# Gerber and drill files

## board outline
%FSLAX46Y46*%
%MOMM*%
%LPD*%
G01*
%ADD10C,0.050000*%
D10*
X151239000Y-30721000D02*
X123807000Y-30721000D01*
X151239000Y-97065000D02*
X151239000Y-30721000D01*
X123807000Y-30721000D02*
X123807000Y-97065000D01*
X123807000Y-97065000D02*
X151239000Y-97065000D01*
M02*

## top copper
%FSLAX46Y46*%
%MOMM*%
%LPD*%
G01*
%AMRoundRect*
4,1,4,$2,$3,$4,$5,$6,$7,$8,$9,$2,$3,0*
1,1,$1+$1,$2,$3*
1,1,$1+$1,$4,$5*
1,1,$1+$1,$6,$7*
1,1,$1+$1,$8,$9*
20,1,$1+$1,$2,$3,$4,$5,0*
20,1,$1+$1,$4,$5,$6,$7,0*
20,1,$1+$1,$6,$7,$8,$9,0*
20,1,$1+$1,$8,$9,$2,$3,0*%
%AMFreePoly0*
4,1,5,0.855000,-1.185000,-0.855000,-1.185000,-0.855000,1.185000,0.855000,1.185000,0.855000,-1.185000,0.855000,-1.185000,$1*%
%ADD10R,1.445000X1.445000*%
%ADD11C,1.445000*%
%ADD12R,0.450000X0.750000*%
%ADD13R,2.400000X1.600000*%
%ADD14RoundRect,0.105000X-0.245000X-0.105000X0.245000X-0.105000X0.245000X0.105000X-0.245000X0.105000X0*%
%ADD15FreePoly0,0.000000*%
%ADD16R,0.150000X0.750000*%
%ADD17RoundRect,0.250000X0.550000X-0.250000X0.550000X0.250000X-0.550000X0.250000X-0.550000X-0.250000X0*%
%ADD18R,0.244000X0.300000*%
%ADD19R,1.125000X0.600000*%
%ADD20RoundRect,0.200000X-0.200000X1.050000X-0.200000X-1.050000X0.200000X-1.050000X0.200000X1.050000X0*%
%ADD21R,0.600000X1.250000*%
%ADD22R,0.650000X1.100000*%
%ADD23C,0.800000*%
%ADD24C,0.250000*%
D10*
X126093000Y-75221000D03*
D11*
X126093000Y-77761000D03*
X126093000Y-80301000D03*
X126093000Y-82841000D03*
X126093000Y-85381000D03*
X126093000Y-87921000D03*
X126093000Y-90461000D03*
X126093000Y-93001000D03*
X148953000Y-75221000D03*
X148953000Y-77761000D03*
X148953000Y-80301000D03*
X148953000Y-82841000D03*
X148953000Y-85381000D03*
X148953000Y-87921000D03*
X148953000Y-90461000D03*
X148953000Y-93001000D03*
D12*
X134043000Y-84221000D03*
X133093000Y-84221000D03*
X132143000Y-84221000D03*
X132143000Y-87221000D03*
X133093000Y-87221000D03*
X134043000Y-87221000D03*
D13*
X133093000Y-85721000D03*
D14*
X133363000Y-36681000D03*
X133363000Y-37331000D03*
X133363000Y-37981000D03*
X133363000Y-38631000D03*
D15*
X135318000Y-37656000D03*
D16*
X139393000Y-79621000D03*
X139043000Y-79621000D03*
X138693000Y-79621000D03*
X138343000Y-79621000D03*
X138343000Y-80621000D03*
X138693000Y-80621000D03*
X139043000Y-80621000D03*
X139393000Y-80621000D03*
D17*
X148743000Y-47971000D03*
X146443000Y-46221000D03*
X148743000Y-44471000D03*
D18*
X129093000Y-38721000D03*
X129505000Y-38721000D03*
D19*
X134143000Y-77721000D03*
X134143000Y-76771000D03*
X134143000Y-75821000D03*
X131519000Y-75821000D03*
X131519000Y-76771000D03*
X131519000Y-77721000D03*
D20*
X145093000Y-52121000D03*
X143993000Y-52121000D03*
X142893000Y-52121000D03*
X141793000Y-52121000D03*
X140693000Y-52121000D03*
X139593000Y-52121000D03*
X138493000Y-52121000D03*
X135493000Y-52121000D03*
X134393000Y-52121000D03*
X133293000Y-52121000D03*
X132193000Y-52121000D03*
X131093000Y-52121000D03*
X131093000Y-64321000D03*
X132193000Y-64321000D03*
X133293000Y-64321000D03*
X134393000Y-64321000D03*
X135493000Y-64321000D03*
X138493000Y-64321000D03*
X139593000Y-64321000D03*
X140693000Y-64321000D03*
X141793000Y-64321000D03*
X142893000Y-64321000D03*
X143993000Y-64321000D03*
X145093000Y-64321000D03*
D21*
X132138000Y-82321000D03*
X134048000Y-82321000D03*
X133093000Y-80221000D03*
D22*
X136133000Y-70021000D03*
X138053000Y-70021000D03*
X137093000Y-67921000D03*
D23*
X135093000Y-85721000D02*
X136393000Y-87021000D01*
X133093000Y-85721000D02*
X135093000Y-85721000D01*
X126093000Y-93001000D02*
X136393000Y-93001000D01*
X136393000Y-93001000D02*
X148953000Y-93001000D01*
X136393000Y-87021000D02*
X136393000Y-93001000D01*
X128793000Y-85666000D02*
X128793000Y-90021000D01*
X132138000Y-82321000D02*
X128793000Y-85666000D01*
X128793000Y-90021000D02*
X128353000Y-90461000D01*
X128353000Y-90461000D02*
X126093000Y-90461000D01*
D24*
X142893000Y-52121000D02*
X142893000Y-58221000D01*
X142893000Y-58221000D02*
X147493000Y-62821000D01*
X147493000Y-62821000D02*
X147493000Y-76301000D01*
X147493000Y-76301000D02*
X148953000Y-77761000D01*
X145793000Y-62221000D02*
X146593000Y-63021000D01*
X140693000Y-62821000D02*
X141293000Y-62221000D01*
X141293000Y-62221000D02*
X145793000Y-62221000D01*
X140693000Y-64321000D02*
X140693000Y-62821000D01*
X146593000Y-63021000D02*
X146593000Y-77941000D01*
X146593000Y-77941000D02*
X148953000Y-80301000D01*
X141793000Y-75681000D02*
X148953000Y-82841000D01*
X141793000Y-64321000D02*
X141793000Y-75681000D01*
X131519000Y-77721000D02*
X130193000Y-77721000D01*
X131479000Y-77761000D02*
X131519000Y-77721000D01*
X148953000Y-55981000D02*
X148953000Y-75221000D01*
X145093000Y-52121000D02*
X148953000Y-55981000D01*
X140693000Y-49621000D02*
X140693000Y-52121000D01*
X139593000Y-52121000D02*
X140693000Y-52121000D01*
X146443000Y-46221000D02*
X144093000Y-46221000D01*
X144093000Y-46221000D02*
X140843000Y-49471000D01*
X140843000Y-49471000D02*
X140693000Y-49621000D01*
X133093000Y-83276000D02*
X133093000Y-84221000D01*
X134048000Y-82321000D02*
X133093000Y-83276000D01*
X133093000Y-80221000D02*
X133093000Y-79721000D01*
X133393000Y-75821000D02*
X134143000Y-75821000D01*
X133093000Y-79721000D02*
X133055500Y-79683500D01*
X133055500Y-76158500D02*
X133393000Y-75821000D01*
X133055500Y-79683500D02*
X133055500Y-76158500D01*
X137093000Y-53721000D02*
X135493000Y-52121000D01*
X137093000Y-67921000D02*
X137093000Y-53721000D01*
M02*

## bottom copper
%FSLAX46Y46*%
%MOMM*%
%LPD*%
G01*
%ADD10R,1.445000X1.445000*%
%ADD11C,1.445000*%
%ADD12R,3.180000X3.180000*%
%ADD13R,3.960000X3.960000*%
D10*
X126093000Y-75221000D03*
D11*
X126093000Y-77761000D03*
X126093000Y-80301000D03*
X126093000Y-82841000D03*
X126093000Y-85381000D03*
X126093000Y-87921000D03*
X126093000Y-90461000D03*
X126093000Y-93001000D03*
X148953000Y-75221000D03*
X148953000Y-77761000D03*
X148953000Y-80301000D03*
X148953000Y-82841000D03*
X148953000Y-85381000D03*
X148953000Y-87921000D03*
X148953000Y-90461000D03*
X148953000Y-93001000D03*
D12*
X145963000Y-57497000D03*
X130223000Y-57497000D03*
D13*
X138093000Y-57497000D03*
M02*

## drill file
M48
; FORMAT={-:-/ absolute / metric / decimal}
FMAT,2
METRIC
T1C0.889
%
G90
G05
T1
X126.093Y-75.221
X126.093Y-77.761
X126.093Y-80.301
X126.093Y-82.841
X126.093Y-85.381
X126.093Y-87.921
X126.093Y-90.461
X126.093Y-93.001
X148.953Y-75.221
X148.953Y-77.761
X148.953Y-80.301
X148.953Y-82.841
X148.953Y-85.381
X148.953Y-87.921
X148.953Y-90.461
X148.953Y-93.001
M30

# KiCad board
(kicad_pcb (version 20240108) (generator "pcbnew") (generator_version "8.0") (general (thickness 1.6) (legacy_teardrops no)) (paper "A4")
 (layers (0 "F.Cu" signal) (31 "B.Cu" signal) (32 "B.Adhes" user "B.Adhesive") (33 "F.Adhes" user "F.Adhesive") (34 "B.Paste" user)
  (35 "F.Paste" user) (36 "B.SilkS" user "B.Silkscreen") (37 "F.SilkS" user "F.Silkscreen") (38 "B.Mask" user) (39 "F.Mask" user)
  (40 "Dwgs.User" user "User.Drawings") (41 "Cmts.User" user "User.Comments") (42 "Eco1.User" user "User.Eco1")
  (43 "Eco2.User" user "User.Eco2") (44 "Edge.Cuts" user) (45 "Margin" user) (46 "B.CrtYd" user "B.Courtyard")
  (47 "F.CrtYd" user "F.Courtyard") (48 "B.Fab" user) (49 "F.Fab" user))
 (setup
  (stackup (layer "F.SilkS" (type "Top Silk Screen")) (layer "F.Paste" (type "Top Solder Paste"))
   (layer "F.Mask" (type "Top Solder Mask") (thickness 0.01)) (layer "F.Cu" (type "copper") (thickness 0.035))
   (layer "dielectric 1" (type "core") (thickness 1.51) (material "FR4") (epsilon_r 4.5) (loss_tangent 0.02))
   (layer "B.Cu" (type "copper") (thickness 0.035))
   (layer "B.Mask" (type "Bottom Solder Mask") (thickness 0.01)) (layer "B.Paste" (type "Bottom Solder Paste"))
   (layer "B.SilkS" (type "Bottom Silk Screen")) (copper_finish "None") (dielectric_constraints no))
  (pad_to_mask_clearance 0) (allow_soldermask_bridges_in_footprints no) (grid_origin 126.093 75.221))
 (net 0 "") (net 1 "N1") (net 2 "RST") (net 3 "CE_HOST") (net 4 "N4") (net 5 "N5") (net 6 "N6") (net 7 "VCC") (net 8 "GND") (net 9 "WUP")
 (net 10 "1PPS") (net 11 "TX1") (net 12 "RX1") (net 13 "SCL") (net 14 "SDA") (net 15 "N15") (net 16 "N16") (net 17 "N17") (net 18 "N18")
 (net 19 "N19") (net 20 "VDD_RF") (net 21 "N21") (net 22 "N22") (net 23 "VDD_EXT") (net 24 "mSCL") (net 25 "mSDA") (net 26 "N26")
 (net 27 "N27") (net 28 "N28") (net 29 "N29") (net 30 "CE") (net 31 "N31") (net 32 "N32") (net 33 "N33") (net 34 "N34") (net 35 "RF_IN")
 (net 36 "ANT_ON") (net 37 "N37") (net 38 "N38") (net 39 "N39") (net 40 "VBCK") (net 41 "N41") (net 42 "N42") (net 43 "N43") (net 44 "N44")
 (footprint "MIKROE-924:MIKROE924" (layer "F.Cu") (at 126.093 75.221)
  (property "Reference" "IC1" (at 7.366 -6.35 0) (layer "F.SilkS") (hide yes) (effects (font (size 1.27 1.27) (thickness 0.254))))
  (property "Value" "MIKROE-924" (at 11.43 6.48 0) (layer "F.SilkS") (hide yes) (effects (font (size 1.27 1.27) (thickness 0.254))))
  (pad "1" thru_hole rect (at 0 0 90) (size 1.445 1.445) (drill 0.889) (layers "*.Cu" "*.Mask" "F.SilkS") (remove_unused_layers no)
   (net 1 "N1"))
  (pad "2" thru_hole circle (at 0 2.54 90) (size 1.445 1.445) (drill 0.889) (layers "*.Cu" "*.Mask" "F.SilkS") (remove_unused_layers no)
   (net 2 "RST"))
  (pad "3" thru_hole circle (at 0 5.08 90) (size 1.445 1.445) (drill 0.889) (layers "*.Cu" "*.Mask" "F.SilkS") (remove_unused_layers no)
   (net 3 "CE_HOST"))
  (pad "4" thru_hole circle (at 0 7.62 90) (size 1.445 1.445) (drill 0.889) (layers "*.Cu" "*.Mask" "F.SilkS") (remove_unused_layers no)
   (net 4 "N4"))
  (pad "5" thru_hole circle (at 0 10.16 90) (size 1.445 1.445) (drill 0.889) (layers "*.Cu" "*.Mask" "F.SilkS") (remove_unused_layers no)
   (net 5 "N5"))
  (pad "6" thru_hole circle (at 0 12.7 90) (size 1.445 1.445) (drill 0.889) (layers "*.Cu" "*.Mask" "F.SilkS") (remove_unused_layers no)
   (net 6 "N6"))
  (pad "7" thru_hole circle (at 0 15.24 90) (size 1.445 1.445) (drill 0.889) (layers "*.Cu" "*.Mask" "F.SilkS") (remove_unused_layers no)
   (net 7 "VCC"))
  (pad "8" thru_hole circle (at 0 17.78 90) (size 1.445 1.445) (drill 0.889) (layers "*.Cu" "*.Mask" "F.SilkS") (remove_unused_layers no)
   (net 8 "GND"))
  (pad "9" thru_hole circle (at 22.86 0 90) (size 1.445 1.445) (drill 0.889) (layers "*.Cu" "*.Mask" "F.SilkS") (remove_unused_layers no)
   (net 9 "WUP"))
  (pad "10" thru_hole circle (at 22.86 2.54 90) (size 1.445 1.445) (drill 0.889) (layers "*.Cu" "*.Mask" "F.SilkS")
   (remove_unused_layers no) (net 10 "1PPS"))
  (pad "11" thru_hole circle (at 22.86 5.08 90) (size 1.445 1.445) (drill 0.889) (layers "*.Cu" "*.Mask" "F.SilkS")
   (remove_unused_layers no) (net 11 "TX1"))
  (pad "12" thru_hole circle (at 22.86 7.62 90) (size 1.445 1.445) (drill 0.889) (layers "*.Cu" "*.Mask" "F.SilkS")
   (remove_unused_layers no) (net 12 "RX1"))
  (pad "13" thru_hole circle (at 22.86 10.16 90) (size 1.445 1.445) (drill 0.889) (layers "*.Cu" "*.Mask" "F.SilkS")
   (remove_unused_layers no) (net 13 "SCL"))
  (pad "14" thru_hole circle (at 22.86 12.7 90) (size 1.445 1.445) (drill 0.889) (layers "*.Cu" "*.Mask" "F.SilkS")
   (remove_unused_layers no) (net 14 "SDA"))
  (pad "15" thru_hole circle (at 22.86 15.24 90) (size 1.445 1.445) (drill 0.889) (layers "*.Cu" "*.Mask" "F.SilkS")
   (remove_unused_layers no) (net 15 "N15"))
  (pad "16" thru_hole circle (at 22.86 17.78 90) (size 1.445 1.445) (drill 0.889) (layers "*.Cu" "*.Mask" "F.SilkS")
   (remove_unused_layers no) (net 8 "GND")))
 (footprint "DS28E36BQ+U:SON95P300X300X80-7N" (layer "F.Cu") (at 133.093 85.721 -90)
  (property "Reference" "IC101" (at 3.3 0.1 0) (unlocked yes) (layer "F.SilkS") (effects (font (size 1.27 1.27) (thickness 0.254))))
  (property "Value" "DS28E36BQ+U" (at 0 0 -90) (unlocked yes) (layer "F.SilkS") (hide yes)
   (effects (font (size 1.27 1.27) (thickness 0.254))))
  (pad "1" smd rect (at -1.5 -0.95) (size 0.45 0.75) (layers "F.Cu" "F.Paste" "F.Mask") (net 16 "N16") (thermal_bridge_angle 45))
  (pad "2" smd rect (at -1.5 0) (size 0.45 0.75) (layers "F.Cu" "F.Paste" "F.Mask") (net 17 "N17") (thermal_bridge_angle 45))
  (pad "3" smd rect (at -1.5 0.95) (size 0.45 0.75) (layers "F.Cu" "F.Paste" "F.Mask") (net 8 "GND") (thermal_bridge_angle 45))
  (pad "4" smd rect (at 1.5 0.95) (size 0.45 0.75) (layers "F.Cu" "F.Paste" "F.Mask") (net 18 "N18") (thermal_bridge_angle 45))
  (pad "5" smd rect (at 1.5 0) (size 0.45 0.75) (layers "F.Cu" "F.Paste" "F.Mask") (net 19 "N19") (thermal_bridge_angle 45))
  (pad "6" smd rect (at 1.5 -0.95) (size 0.45 0.75) (layers "F.Cu" "F.Paste" "F.Mask") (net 7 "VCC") (thermal_bridge_angle 45))
  (pad "7" smd rect (at 0 0 270) (size 1.6 2.4) (layers "F.Cu" "F.Paste" "F.Mask") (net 8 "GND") (thermal_bridge_angle 45)))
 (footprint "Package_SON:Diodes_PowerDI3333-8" (layer "F.Cu") (at 134.863 37.656)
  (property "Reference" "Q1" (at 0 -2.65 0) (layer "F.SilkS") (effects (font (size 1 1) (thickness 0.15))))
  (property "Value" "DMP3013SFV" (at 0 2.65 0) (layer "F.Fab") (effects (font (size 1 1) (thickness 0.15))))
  (pad "" smd roundrect (at 0.02 -0.565) (size 0.6 1) (layers "F.Paste") (roundrect_rratio 0.25) (solder_paste_margin_ratio -0.2))
  (pad "" smd roundrect (at 0.02 0.565) (size 0.6 1) (layers "F.Paste") (roundrect_rratio 0.25) (solder_paste_margin_ratio -0.2))
  (pad "" smd roundrect (at 0.73 -0.565) (size 0.6 1) (layers "F.Paste") (roundrect_rratio 0.25) (solder_paste_margin_ratio -0.2))
  (pad "" smd roundrect (at 0.73 0.565) (size 0.6 1) (layers "F.Paste") (roundrect_rratio 0.25) (solder_paste_margin_ratio -0.2))
  (pad "" smd roundrect (at 1.5 -0.975) (size 0.7 0.42) (layers "F.Paste") (roundrect_rratio 0.25))
  (pad "" smd roundrect (at 1.5 -0.325) (size 0.7 0.42) (layers "F.Paste") (roundrect_rratio 0.25))
  (pad "" smd roundrect (at 1.5 0.325) (size 0.7 0.42) (layers "F.Paste") (roundrect_rratio 0.25))
  (pad "" smd roundrect (at 1.5 0.975) (size 0.7 0.42) (layers "F.Paste") (roundrect_rratio 0.25))
  (pad "1" smd roundrect (at -1.5 -0.975) (size 0.7 0.42) (layers "F.Cu" "F.Paste" "F.Mask") (roundrect_rratio 0.25) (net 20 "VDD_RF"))
  (pad "2" smd roundrect (at -1.5 -0.325) (size 0.7 0.42) (layers "F.Cu" "F.Paste" "F.Mask") (roundrect_rratio 0.25) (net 20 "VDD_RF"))
  (pad "3" smd roundrect (at -1.5 0.325) (size 0.7 0.42) (layers "F.Cu" "F.Paste" "F.Mask") (roundrect_rratio 0.25) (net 20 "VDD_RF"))
  (pad "4" smd roundrect (at -1.5 0.975) (size 0.7 0.42) (layers "F.Cu" "F.Paste" "F.Mask") (roundrect_rratio 0.25) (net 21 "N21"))
  (pad "5" smd custom (at 0.455 0) (size 1.71 2.37) (layers "F.Cu" "F.Mask") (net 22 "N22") (thermal_bridge_angle 45)
   (options (clearance outline) (anchor rect)) (primitives)))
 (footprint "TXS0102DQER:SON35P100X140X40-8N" (layer "F.Cu") (at 138.868 80.121 -90)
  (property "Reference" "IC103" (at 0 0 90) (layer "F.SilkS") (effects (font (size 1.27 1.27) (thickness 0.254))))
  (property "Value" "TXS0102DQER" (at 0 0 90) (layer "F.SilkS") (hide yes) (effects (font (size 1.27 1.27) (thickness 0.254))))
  (pad "1" smd rect (at -0.5 -0.525) (size 0.15 0.75) (layers "F.Cu" "F.Paste" "F.Mask") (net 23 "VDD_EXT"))
  (pad "2" smd rect (at -0.5 -0.175) (size 0.15 0.75) (layers "F.Cu" "F.Paste" "F.Mask") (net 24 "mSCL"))
  (pad "3" smd rect (at -0.5 0.175) (size 0.15 0.75) (layers "F.Cu" "F.Paste" "F.Mask") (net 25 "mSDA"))
  (pad "4" smd rect (at -0.5 0.525) (size 0.15 0.75) (layers "F.Cu" "F.Paste" "F.Mask") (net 8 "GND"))
  (pad "5" smd rect (at 0.5 0.525) (size 0.15 0.75) (layers "F.Cu" "F.Paste" "F.Mask") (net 23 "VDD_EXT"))
  (pad "6" smd rect (at 0.5 0.175) (size 0.15 0.75) (layers "F.Cu" "F.Paste" "F.Mask") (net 14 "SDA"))
  (pad "7" smd rect (at 0.5 -0.175) (size 0.15 0.75) (layers "F.Cu" "F.Paste" "F.Mask") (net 13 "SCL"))
  (pad "8" smd rect (at 0.5 -0.525) (size 0.15 0.75) (layers "F.Cu" "F.Paste" "F.Mask") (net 7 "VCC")))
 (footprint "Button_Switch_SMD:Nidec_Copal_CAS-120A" (layer "F.Cu") (at 147.593 46.221 180)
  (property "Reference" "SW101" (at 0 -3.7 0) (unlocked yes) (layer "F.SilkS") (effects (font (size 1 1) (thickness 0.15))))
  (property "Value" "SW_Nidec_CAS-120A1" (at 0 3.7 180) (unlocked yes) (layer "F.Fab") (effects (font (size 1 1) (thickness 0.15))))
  (pad "1" smd roundrect (at -1.15 -1.75 90) (size 1 1.6) (layers "F.Cu" "F.Paste" "F.Mask") (roundrect_rratio 0.25) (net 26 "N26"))
  (pad "2" smd roundrect (at 1.15 0 90) (size 1 1.6) (layers "F.Cu" "F.Paste" "F.Mask") (roundrect_rratio 0.25) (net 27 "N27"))
  (pad "3" smd roundrect (at -1.15 1.75 90) (size 1 1.6) (layers "F.Cu" "F.Paste" "F.Mask") (roundrect_rratio 0.25) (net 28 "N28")))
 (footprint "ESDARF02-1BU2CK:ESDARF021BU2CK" (layer "F.Cu") (at 129.299 38.721)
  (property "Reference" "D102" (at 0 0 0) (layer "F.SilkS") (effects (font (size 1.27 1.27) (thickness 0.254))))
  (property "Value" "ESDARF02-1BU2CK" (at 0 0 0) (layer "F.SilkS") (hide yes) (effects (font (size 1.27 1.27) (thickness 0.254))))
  (pad "1" smd rect (at -0.206 0) (size 0.244 0.3) (layers "F.Cu" "F.Paste" "F.Mask") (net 8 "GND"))
  (pad "2" smd rect (at 0.206 0) (size 0.244 0.3) (layers "F.Cu" "F.Paste" "F.Mask") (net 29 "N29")))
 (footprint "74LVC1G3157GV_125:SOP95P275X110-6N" (layer "F.Cu") (at 132.831 76.771 180)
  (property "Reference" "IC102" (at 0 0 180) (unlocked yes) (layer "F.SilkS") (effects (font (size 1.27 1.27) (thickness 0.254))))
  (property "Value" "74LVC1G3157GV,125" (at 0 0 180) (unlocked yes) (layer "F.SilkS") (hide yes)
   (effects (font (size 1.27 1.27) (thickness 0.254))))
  (pad "1" smd rect (at -1.312 -0.95 270) (size 0.6 1.125) (layers "F.Cu" "F.Paste" "F.Mask") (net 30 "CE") (thermal_bridge_angle 45))
  (pad "2" smd rect (at -1.312 0 270) (size 0.6 1.125) (layers "F.Cu" "F.Paste" "F.Mask") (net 8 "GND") (thermal_bridge_angle 45))
  (pad "3" smd rect (at -1.312 0.95 270) (size 0.6 1.125) (layers "F.Cu" "F.Paste" "F.Mask") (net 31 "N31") (thermal_bridge_angle 45))
  (pad "4" smd rect (at 1.312 0.95 270) (size 0.6 1.125) (layers "F.Cu" "F.Paste" "F.Mask") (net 3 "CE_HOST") (thermal_bridge_angle 45))
  (pad "5" smd rect (at 1.312 0 270) (size 0.6 1.125) (layers "F.Cu" "F.Paste" "F.Mask") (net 7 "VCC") (thermal_bridge_angle 45))
  (pad "6" smd rect (at 1.312 -0.95 270) (size 0.6 1.125) (layers "F.Cu" "F.Paste" "F.Mask") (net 2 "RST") (thermal_bridge_angle 45)))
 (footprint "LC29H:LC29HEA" (layer "F.Cu") (at 138.093 58.221 -90)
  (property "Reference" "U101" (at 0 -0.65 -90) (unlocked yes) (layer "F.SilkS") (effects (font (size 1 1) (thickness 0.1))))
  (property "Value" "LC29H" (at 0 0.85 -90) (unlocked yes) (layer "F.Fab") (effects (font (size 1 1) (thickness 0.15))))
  (pad "1" smd roundrect (at -6.1 -7 270) (size 2.5 0.8) (layers "F.Cu" "F.Paste" "F.Mask") (roundrect_rratio 0.25) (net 9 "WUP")
   (thermal_bridge_angle 45))
  (pad "2" smd roundrect (at -6.1 -5.9 270) (size 2.5 0.8) (layers "F.Cu" "F.Paste" "F.Mask") (roundrect_rratio 0.25) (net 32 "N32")
   (thermal_bridge_angle 45))
  (pad "3" smd roundrect (at -6.1 -4.8 270) (size 2.5 0.8) (layers "F.Cu" "F.Paste" "F.Mask") (roundrect_rratio 0.25) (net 10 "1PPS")
   (thermal_bridge_angle 45))
  (pad "4" smd roundrect (at -6.1 -3.7 270) (size 2.5 0.8) (layers "F.Cu" "F.Paste" "F.Mask") (roundrect_rratio 0.25) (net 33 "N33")
   (thermal_bridge_angle 45))
  (pad "5" smd roundrect (at -6.1 -2.6 270) (size 2.5 0.8) (layers "F.Cu" "F.Paste" "F.Mask") (roundrect_rratio 0.25) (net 27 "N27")
   (thermal_bridge_angle 45))
  (pad "6" smd roundrect (at -6.1 -1.5 270) (size 2.5 0.8) (layers "F.Cu" "F.Paste" "F.Mask") (roundrect_rratio 0.25) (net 27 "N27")
   (thermal_bridge_angle 45))
  (pad "7" smd roundrect (at -6.1 -0.4 270) (size 2.5 0.8) (layers "F.Cu" "F.Paste" "F.Mask") (roundrect_rratio 0.25) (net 23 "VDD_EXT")
   (thermal_bridge_angle 45))
  (pad "8" smd roundrect (at -6.1 2.6 270) (size 2.5 0.8) (layers "F.Cu" "F.Paste" "F.Mask") (roundrect_rratio 0.25) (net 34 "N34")
   (thermal_bridge_angle 45))
  (pad "9" smd roundrect (at -6.1 3.7 270) (size 2.5 0.8) (layers "F.Cu" "F.Paste" "F.Mask") (roundrect_rratio 0.25) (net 20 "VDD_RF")
   (thermal_bridge_angle 45))
  (pad "10" smd roundrect (at -6.1 4.8 270) (size 2.5 0.8) (layers "F.Cu" "F.Paste" "F.Mask") (roundrect_rratio 0.25) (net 8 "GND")
   (thermal_bridge_angle 45))
  (pad "11" smd roundrect (at -6.1 5.9 270) (size 2.5 0.8) (layers "F.Cu" "F.Paste" "F.Mask") (roundrect_rratio 0.25) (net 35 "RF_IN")
   (thermal_bridge_angle 45))
  (pad "12" smd roundrect (at -6.1 7 270) (size 2.5 0.8) (layers "F.Cu" "F.Paste" "F.Mask") (roundrect_rratio 0.25) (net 8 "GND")
   (thermal_bridge_angle 45))
  (pad "13" smd roundrect (at 6.1 7 270) (size 2.5 0.8) (layers "F.Cu" "F.Paste" "F.Mask") (roundrect_rratio 0.25) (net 8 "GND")
   (thermal_bridge_angle 45))
  (pad "14" smd roundrect (at 6.1 5.9 270) (size 2.5 0.8) (layers "F.Cu" "F.Paste" "F.Mask") (roundrect_rratio 0.25) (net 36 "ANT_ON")
   (thermal_bridge_angle 45))
  (pad "15" smd roundrect (at 6.1 4.8 270) (size 2.5 0.8) (layers "F.Cu" "F.Paste" "F.Mask") (roundrect_rratio 0.25) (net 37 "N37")
   (thermal_bridge_angle 45))
  (pad "16" smd roundrect (at 6.1 3.7 270) (size 2.5 0.8) (layers "F.Cu" "F.Paste" "F.Mask") (roundrect_rratio 0.25) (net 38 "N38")
   (thermal_bridge_angle 45))
  (pad "17" smd roundrect (at 6.1 2.6 270) (size 2.5 0.8) (layers "F.Cu" "F.Paste" "F.Mask") (roundrect_rratio 0.25) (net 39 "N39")
   (thermal_bridge_angle 45))
  (pad "18" smd roundrect (at 6.1 -0.4 270) (size 2.5 0.8) (layers "F.Cu" "F.Paste" "F.Mask") (roundrect_rratio 0.25) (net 25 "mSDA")
   (thermal_bridge_angle 45))
  (pad "19" smd roundrect (at 6.1 -1.5 270) (size 2.5 0.8) (layers "F.Cu" "F.Paste" "F.Mask") (roundrect_rratio 0.25) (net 24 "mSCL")
   (thermal_bridge_angle 45))
  (pad "20" smd roundrect (at 6.1 -2.6 270) (size 2.5 0.8) (layers "F.Cu" "F.Paste" "F.Mask") (roundrect_rratio 0.25) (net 11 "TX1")
   (thermal_bridge_angle 45))
  (pad "21" smd roundrect (at 6.1 -3.7 270) (size 2.5 0.8) (layers "F.Cu" "F.Paste" "F.Mask") (roundrect_rratio 0.25) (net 12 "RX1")
   (thermal_bridge_angle 45))
  (pad "22" smd roundrect (at 6.1 -4.8 270) (size 2.5 0.8) (layers "F.Cu" "F.Paste" "F.Mask") (roundrect_rratio 0.25) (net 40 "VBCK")
   (thermal_bridge_angle 45))
  (pad "23" smd roundrect (at 6.1 -5.9 270) (size 2.5 0.8) (layers "F.Cu" "F.Paste" "F.Mask") (roundrect_rratio 0.25) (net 7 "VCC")
   (thermal_bridge_angle 45))
  (pad "24" smd roundrect (at 6.1 -7 270) (size 2.5 0.8) (layers "F.Cu" "F.Paste" "F.Mask") (roundrect_rratio 0.25) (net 8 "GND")
   (thermal_bridge_angle 45)))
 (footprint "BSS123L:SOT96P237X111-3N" (layer "F.Cu") (at 133.093 81.271 90)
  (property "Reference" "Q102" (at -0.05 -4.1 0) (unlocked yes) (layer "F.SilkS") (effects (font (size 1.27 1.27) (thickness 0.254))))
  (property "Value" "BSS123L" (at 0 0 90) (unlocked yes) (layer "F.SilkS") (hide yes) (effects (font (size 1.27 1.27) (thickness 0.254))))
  (pad "1" smd rect (at -1.05 -0.955 180) (size 0.6 1.25) (layers "F.Cu" "F.Paste" "F.Mask") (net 7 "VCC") (thermal_bridge_angle 45))
  (pad "2" smd rect (at -1.05 0.955 180) (size 0.6 1.25) (layers "F.Cu" "F.Paste" "F.Mask") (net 17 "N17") (thermal_bridge_angle 45))
  (pad "3" smd rect (at 1.05 0 180) (size 0.6 1.25) (layers "F.Cu" "F.Paste" "F.Mask") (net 31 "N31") (thermal_bridge_angle 45)))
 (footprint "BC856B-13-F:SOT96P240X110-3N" (layer "F.Cu") (at 137.093 68.971 90)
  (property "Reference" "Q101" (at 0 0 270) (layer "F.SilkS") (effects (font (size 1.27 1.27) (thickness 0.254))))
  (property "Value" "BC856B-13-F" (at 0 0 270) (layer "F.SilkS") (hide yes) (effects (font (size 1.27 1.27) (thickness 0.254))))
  (pad "1" smd rect (at -1.05 -0.96 180) (size 0.65 1.1) (layers "F.Cu" "F.Paste" "F.Mask") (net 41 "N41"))
  (pad "2" smd rect (at -1.05 0.96 180) (size 0.65 1.1) (layers "F.Cu" "F.Paste" "F.Mask") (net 8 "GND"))
  (pad "3" smd rect (at 1.05 0 180) (size 0.65 1.1) (layers "F.Cu" "F.Paste" "F.Mask") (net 34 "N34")))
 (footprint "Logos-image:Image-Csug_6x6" (layer "B.Cu") (at 128.379 70.141 180)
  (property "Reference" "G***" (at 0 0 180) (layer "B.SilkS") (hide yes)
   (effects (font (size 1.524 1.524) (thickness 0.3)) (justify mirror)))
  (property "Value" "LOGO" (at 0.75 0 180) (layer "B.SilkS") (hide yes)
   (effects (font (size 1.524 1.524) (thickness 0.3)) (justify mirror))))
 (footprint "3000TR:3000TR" (layer "B.Cu") (at 138.093 58.221 180)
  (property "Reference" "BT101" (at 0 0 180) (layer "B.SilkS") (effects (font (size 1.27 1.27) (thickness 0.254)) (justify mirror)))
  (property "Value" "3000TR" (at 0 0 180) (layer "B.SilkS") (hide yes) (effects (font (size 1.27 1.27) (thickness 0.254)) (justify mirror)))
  (pad "1" smd rect (at -7.87 0.724 90) (size 3.18 3.18) (layers "B.Cu" "B.Paste" "B.Mask") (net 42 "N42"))
  (pad "2" smd rect (at 7.87 0.724 90) (size 3.18 3.18) (layers "B.Cu" "B.Paste" "B.Mask") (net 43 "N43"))
  (pad "3" smd rect (at 0 0.724 90) (size 3.96 3.96) (layers "B.Cu" "B.Paste" "B.Mask") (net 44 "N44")))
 (gr_line (start 151.239 30.721) (end 123.807 30.721) (stroke (width 0.05) (type solid)) (layer "Edge.Cuts"))
 (gr_line (start 151.239 97.065) (end 151.239 30.721) (stroke (width 0.05) (type solid)) (layer "Edge.Cuts"))
 (gr_line (start 123.807 30.721) (end 123.807 97.065) (stroke (width 0.05) (type solid)) (layer "Edge.Cuts"))
 (gr_line (start 123.807 97.065) (end 151.239 97.065) (stroke (width 0.05) (type solid)) (layer "Edge.Cuts"))
 (segment (start 135.093 85.721) (end 136.393 87.021) (width 0.8) (layer "F.Cu") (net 8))
 (segment (start 133.093 85.721) (end 135.093 85.721) (width 0.8) (layer "F.Cu") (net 8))
 (segment (start 126.093 93.001) (end 136.393 93.001) (width 0.8) (layer "F.Cu") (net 8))
 (segment (start 136.393 93.001) (end 148.953 93.001) (width 0.8) (layer "F.Cu") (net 8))
 (segment (start 136.393 87.021) (end 136.393 93.001) (width 0.8) (layer "F.Cu") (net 8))
 (segment (start 128.793 85.666) (end 128.793 90.021) (width 0.8) (layer "F.Cu") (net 7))
 (segment (start 132.138 82.321) (end 128.793 85.666) (width 0.8) (layer "F.Cu") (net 7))
 (segment (start 128.793 90.021) (end 128.353 90.461) (width 0.8) (layer "F.Cu") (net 7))
 (segment (start 128.353 90.461) (end 126.093 90.461) (width 0.8) (layer "F.Cu") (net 7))
 (segment (start 142.893 52.121) (end 142.893 58.221) (width 0.25) (layer "F.Cu") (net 10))
 (segment (start 142.893 58.221) (end 147.493 62.821) (width 0.25) (layer "F.Cu") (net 10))
 (segment (start 147.493 62.821) (end 147.493 76.301) (width 0.25) (layer "F.Cu") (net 10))
 (segment (start 147.493 76.301) (end 148.953 77.761) (width 0.25) (layer "F.Cu") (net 10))
 (segment (start 145.793 62.221) (end 146.593 63.021) (width 0.25) (layer "F.Cu") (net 11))
 (segment (start 140.693 62.821) (end 141.293 62.221) (width 0.25) (layer "F.Cu") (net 11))
 (segment (start 141.293 62.221) (end 145.793 62.221) (width 0.25) (layer "F.Cu") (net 11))
 (segment (start 140.693 64.321) (end 140.693 62.821) (width 0.25) (layer "F.Cu") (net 11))
 (segment (start 146.593 63.021) (end 146.593 77.941) (width 0.25) (layer "F.Cu") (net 11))
 (segment (start 146.593 77.941) (end 148.953 80.301) (width 0.25) (layer "F.Cu") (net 11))
 (segment (start 141.793 75.681) (end 148.953 82.841) (width 0.25) (layer "F.Cu") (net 12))
 (segment (start 141.793 64.321) (end 141.793 75.681) (width 0.25) (layer "F.Cu") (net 12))
 (segment (start 131.519 77.721) (end 130.193 77.721) (width 0.25) (layer "F.Cu") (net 2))
 (segment (start 131.479 77.761) (end 131.519 77.721) (width 0.25) (layer "F.Cu") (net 2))
 (segment (start 148.953 55.981) (end 148.953 75.221) (width 0.25) (layer "F.Cu") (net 9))
 (segment (start 145.093 52.121) (end 148.953 55.981) (width 0.25) (layer "F.Cu") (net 9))
 (segment (start 140.693 49.621) (end 140.693 52.121) (width 0.25) (layer "F.Cu") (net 27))
 (segment (start 139.593 52.121) (end 140.693 52.121) (width 0.25) (layer "F.Cu") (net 27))
 (segment (start 146.443 46.221) (end 144.093 46.221) (width 0.25) (layer "F.Cu") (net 27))
 (segment (start 144.093 46.221) (end 140.843 49.471) (width 0.25) (layer "F.Cu") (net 27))
 (segment (start 140.843 49.471) (end 140.693 49.621) (width 0.25) (layer "F.Cu") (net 27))
 (segment (start 133.093 83.276) (end 133.093 84.221) (width 0.25) (layer "F.Cu") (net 17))
 (segment (start 134.048 82.321) (end 133.093 83.276) (width 0.25) (layer "F.Cu") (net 17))
 (segment (start 133.093 80.221) (end 133.093 79.721) (width 0.25) (layer "F.Cu") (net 31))
 (segment (start 133.393 75.821) (end 134.143 75.821) (width 0.25) (layer "F.Cu") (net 31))
 (segment (start 133.093 79.721) (end 133.0555 79.6835) (width 0.25) (layer "F.Cu") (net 31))
 (segment (start 133.0555 76.1585) (end 133.393 75.821) (width 0.25) (layer "F.Cu") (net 31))
 (segment (start 133.0555 79.6835) (end 133.0555 76.1585) (width 0.25) (layer "F.Cu") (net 31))
 (segment (start 137.093 53.721) (end 135.493 52.121) (width 0.25) (layer "F.Cu") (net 34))
 (segment (start 137.093 67.921) (end 137.093 53.721) (width 0.25) (layer "F.Cu") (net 34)))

